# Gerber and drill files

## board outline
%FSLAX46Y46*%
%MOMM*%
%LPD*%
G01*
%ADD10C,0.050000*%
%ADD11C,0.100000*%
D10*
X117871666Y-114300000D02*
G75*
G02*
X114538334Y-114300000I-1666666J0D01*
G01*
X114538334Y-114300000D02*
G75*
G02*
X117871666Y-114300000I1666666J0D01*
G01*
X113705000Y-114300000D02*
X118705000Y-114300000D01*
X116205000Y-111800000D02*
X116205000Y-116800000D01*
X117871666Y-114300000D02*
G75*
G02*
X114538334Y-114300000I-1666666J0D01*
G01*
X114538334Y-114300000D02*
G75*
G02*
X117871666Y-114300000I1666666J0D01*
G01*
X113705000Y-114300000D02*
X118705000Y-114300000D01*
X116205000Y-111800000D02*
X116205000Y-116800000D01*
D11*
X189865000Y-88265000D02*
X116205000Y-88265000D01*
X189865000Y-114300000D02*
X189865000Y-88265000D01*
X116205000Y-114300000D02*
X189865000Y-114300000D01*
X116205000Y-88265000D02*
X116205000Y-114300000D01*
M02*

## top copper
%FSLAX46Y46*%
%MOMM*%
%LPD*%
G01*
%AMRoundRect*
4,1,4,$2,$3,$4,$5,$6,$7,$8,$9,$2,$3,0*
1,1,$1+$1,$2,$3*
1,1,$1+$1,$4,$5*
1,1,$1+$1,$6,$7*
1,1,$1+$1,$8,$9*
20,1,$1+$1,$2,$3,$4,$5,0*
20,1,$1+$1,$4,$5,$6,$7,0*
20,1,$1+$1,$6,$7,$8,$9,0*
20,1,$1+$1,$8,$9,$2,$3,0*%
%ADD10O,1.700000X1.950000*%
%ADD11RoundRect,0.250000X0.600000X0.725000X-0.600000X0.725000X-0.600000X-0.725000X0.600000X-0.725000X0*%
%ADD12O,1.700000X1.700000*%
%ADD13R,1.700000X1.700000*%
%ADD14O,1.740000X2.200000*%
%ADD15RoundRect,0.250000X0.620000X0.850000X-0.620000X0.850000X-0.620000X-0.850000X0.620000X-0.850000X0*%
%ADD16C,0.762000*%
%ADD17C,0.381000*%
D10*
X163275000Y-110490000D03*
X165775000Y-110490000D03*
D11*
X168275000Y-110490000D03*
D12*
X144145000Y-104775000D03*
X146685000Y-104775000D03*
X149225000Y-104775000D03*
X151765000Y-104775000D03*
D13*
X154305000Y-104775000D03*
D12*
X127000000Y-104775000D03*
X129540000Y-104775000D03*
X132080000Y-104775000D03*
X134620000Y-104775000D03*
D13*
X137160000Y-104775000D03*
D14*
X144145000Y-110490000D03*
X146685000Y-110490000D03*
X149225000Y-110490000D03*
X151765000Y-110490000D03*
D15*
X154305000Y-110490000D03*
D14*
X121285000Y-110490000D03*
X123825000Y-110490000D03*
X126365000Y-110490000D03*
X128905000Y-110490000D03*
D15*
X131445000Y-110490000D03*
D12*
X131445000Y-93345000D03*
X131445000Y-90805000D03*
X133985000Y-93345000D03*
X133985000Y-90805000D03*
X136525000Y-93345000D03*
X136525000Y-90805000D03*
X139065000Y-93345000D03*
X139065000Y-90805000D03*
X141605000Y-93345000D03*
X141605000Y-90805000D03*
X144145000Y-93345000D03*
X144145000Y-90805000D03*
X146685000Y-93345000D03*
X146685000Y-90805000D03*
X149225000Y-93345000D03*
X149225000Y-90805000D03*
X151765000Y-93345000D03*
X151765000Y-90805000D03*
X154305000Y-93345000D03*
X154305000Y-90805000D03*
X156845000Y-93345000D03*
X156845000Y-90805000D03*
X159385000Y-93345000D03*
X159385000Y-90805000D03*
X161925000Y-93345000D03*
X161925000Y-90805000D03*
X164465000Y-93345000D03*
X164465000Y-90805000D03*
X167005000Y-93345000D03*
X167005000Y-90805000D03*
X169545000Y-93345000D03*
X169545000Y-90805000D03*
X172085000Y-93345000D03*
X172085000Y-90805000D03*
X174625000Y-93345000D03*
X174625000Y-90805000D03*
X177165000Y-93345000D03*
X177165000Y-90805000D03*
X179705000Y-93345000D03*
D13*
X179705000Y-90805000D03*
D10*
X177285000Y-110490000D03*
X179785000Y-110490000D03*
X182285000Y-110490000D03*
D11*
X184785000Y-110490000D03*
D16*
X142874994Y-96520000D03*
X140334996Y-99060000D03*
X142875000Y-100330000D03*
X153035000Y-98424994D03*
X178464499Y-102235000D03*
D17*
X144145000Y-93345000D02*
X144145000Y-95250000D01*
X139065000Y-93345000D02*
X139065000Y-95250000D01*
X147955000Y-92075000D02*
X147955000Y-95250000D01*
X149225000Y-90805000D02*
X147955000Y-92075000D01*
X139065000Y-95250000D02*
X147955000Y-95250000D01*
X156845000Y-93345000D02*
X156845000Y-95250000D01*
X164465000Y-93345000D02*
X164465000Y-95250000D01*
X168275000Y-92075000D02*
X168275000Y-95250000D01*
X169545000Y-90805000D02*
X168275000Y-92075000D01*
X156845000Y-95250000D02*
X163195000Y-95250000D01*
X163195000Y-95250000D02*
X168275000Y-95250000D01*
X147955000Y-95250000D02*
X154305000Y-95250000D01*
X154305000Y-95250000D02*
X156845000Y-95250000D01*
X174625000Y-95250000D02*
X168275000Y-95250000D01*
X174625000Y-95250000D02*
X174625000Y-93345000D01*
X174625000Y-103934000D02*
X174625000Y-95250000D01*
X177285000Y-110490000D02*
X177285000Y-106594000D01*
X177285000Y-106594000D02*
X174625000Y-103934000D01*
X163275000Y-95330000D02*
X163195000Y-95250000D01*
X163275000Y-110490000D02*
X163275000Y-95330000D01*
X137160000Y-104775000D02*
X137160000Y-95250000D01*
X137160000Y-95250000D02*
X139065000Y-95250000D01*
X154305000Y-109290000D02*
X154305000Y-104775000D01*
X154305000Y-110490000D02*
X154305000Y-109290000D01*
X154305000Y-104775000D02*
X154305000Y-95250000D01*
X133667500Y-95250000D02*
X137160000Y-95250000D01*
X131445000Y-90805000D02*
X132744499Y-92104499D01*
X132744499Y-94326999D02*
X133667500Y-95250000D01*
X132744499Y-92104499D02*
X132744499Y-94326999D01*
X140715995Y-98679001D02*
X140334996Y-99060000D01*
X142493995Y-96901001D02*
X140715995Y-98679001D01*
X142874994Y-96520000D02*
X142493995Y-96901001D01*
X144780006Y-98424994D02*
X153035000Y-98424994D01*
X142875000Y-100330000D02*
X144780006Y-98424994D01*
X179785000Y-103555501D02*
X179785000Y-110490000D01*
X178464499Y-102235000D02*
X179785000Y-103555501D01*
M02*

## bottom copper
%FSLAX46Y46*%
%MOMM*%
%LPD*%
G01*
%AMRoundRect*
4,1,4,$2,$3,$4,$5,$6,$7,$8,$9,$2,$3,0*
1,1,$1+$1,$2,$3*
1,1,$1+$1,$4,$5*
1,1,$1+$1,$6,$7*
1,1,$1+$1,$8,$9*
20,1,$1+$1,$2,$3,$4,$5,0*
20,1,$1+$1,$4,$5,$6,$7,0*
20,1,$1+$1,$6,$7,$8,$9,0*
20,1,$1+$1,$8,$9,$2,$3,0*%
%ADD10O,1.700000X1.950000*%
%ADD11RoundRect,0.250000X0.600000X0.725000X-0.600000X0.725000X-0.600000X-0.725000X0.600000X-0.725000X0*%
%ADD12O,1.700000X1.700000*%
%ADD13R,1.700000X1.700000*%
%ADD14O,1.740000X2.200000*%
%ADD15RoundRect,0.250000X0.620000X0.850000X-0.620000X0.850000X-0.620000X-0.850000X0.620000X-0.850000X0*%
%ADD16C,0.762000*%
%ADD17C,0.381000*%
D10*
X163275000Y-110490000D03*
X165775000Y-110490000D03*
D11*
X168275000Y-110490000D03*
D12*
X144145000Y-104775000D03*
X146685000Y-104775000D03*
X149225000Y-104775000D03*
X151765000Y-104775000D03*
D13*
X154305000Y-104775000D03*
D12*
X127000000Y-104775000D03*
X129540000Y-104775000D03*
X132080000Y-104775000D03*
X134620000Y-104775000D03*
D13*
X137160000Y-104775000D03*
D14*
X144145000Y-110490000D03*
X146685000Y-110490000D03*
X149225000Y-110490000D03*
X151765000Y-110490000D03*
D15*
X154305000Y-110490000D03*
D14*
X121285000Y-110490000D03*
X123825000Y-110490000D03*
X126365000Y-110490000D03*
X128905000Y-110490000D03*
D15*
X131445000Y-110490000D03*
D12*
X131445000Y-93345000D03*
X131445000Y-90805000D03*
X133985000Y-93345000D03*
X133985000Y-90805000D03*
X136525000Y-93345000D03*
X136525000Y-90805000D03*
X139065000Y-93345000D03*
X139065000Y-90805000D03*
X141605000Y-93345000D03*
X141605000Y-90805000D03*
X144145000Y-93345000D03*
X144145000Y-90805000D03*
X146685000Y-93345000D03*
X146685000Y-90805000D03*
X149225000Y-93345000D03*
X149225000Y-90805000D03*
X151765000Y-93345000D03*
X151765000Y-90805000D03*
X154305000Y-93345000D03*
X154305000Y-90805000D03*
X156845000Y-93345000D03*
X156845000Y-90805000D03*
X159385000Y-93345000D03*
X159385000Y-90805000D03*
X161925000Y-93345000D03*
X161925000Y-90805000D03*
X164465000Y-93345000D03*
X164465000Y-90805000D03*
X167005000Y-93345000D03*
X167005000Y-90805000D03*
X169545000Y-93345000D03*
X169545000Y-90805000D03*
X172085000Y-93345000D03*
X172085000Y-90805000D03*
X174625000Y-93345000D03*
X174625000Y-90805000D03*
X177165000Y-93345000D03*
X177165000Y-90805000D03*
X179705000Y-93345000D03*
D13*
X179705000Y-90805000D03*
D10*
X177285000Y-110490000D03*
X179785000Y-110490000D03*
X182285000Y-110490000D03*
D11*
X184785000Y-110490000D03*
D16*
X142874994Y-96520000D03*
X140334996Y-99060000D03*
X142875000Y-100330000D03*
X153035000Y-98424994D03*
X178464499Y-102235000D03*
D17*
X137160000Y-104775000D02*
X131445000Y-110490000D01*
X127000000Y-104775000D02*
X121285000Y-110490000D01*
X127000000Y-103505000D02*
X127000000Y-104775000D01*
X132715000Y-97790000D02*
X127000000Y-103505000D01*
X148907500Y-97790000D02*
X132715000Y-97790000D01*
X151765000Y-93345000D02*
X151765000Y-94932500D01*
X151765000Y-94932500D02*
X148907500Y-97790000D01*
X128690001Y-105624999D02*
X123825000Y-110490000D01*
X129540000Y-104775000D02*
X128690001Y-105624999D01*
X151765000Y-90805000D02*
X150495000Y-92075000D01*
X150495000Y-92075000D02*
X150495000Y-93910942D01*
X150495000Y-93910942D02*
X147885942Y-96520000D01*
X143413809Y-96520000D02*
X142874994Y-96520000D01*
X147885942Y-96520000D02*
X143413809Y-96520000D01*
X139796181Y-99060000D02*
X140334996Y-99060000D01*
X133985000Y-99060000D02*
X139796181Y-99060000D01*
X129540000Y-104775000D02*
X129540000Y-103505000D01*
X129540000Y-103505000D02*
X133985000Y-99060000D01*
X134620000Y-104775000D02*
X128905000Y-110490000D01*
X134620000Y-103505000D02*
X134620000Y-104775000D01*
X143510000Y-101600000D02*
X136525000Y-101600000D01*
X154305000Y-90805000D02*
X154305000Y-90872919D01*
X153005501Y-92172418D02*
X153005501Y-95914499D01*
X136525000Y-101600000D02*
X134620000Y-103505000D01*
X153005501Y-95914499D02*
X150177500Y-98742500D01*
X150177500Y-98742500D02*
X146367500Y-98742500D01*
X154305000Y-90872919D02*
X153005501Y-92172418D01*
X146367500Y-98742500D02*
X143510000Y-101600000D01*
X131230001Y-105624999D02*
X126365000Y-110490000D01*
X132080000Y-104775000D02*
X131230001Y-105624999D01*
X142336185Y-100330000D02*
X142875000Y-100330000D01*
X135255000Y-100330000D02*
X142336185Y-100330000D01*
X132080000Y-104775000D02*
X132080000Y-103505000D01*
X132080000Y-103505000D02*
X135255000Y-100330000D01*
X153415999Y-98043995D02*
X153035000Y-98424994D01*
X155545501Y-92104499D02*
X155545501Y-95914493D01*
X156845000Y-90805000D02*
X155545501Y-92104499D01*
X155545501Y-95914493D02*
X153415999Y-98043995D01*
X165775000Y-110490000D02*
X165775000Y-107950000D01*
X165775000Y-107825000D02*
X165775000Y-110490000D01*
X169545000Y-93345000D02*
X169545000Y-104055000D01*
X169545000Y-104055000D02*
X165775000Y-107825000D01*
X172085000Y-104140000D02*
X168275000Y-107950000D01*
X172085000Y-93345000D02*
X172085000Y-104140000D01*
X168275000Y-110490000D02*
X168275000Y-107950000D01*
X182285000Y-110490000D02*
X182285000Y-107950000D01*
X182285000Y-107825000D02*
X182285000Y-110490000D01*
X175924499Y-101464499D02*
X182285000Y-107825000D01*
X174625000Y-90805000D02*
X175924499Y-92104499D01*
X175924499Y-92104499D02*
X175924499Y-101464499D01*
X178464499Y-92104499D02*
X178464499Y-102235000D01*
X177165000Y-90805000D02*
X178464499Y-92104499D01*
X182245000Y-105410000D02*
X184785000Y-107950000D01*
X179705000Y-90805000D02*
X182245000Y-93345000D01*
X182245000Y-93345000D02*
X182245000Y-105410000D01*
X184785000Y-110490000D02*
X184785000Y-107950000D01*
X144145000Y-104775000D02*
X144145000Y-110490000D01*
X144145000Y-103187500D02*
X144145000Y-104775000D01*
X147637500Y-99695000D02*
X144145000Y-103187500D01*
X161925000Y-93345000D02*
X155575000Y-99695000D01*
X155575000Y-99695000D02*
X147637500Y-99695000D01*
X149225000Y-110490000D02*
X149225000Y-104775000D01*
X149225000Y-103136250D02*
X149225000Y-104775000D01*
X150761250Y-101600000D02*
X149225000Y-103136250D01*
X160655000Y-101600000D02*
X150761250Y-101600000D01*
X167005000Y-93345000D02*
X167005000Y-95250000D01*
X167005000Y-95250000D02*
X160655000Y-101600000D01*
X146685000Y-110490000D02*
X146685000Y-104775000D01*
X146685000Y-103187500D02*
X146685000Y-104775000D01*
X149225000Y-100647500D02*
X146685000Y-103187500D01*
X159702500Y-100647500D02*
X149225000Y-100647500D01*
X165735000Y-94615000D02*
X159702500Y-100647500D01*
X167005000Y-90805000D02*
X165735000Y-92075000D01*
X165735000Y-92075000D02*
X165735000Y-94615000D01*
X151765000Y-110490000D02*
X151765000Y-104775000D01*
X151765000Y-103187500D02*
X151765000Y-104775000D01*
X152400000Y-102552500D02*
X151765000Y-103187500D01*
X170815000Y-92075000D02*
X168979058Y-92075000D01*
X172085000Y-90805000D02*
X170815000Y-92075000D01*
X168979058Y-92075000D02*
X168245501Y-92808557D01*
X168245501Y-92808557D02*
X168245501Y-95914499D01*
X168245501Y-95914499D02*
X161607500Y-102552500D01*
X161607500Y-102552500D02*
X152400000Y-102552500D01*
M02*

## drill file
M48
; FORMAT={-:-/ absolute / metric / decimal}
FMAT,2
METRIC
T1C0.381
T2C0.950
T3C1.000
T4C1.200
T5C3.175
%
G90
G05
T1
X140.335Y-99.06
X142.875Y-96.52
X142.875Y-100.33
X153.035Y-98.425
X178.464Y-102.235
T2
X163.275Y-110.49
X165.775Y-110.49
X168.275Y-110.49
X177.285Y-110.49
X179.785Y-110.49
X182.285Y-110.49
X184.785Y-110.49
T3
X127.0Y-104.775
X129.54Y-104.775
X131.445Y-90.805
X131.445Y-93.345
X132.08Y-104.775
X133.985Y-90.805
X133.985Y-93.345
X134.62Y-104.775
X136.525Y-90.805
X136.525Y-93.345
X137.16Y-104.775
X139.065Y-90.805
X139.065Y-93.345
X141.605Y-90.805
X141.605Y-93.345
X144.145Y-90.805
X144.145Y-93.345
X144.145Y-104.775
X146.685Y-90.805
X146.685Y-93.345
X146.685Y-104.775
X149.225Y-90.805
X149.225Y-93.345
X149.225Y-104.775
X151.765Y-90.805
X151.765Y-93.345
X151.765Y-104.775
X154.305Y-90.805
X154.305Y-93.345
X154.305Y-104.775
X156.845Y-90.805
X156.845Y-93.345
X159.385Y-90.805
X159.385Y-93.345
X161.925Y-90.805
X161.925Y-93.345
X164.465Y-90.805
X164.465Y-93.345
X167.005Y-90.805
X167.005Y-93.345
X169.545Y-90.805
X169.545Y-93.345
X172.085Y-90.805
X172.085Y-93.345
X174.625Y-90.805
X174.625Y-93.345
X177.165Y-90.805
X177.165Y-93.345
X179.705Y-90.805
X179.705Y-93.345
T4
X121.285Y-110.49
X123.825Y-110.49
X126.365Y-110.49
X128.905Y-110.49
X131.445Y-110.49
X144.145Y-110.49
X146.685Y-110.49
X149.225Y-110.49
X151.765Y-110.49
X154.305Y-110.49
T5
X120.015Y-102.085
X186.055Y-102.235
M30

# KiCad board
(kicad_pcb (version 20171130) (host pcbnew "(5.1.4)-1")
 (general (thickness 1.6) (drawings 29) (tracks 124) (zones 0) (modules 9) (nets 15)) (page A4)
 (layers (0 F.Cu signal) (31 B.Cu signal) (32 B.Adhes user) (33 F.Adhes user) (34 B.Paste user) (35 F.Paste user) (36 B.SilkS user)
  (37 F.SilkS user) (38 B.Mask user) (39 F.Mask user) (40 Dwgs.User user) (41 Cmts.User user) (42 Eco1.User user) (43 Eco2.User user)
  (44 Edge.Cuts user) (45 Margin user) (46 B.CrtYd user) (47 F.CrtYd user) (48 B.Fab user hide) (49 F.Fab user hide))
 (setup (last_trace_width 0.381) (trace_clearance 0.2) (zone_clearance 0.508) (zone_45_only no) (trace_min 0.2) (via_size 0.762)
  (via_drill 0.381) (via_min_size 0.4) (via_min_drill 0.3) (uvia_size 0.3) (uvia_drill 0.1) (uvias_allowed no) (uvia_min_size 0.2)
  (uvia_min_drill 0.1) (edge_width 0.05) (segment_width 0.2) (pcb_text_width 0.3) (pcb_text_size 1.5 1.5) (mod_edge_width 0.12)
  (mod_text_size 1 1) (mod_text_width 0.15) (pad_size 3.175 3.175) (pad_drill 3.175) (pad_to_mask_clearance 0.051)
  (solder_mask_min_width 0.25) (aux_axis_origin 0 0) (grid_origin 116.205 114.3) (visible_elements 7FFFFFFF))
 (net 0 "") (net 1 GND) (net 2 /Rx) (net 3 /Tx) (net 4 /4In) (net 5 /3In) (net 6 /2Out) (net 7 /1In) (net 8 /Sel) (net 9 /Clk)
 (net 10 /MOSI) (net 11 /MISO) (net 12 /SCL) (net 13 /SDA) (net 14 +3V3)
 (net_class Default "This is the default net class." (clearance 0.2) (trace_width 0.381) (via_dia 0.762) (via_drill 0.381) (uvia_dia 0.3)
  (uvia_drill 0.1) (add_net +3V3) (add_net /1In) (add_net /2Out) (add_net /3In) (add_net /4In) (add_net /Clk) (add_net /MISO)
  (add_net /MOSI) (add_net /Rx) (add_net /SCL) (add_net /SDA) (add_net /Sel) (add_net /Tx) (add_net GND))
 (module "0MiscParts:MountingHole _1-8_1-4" (layer F.Cu) (at 186.055 102.235 270)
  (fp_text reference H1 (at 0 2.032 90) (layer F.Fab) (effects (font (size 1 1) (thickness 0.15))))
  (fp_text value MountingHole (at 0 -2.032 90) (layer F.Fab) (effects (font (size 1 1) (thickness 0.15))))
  (pad "" np_thru_hole circle (at 0 0 270) (size 3.175 3.175) (drill 3.175) (layers *.Cu *.Mask)))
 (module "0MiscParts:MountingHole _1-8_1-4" (layer F.Cu) (at 120.015 102.085 270)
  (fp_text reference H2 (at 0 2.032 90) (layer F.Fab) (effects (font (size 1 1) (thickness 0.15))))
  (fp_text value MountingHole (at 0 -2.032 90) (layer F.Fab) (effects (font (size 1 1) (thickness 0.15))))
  (pad "" np_thru_hole circle (at 0 0 270) (size 3.175 3.175) (drill 3.175) (layers *.Cu *.Mask)))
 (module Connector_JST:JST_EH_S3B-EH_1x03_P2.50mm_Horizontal (layer F.Cu) (at 168.275 110.49 180)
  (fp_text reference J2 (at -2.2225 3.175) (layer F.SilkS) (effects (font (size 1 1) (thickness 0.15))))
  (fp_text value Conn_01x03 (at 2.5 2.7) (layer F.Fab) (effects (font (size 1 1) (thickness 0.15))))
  (pad 3 thru_hole oval (at 5 0 180) (size 1.7 1.95) (drill 0.95) (layers *.Cu *.Mask) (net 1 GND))
  (pad 2 thru_hole oval (at 2.5 0 180) (size 1.7 1.95) (drill 0.95) (layers *.Cu *.Mask) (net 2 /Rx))
  (pad 1 thru_hole roundrect (at 0 0 180) (size 1.7 1.95) (drill 0.95) (layers *.Cu *.Mask) (roundrect_rratio 0.147059) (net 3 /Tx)))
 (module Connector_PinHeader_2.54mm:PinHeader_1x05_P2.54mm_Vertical (layer F.Cu) (at 154.305 104.775 270)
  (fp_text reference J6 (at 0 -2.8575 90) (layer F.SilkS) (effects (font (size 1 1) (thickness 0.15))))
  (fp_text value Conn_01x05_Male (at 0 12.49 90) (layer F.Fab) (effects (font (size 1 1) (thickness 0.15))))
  (pad 5 thru_hole oval (at 0 10.16 270) (size 1.7 1.7) (drill 1) (layers *.Cu *.Mask) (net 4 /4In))
  (pad 4 thru_hole oval (at 0 7.62 270) (size 1.7 1.7) (drill 1) (layers *.Cu *.Mask) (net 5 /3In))
  (pad 3 thru_hole oval (at 0 5.08 270) (size 1.7 1.7) (drill 1) (layers *.Cu *.Mask) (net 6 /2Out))
  (pad 2 thru_hole oval (at 0 2.54 270) (size 1.7 1.7) (drill 1) (layers *.Cu *.Mask) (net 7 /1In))
  (pad 1 thru_hole rect (at 0 0 270) (size 1.7 1.7) (drill 1) (layers *.Cu *.Mask) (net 1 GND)))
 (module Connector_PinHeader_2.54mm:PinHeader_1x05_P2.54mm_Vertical (layer F.Cu) (at 137.16 104.775 270)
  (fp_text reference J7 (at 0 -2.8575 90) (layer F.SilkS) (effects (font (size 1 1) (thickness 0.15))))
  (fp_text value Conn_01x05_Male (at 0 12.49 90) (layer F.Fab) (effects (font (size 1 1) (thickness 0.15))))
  (pad 5 thru_hole oval (at 0 10.16 270) (size 1.7 1.7) (drill 1) (layers *.Cu *.Mask) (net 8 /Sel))
  (pad 4 thru_hole oval (at 0 7.62 270) (size 1.7 1.7) (drill 1) (layers *.Cu *.Mask) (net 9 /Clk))
  (pad 3 thru_hole oval (at 0 5.08 270) (size 1.7 1.7) (drill 1) (layers *.Cu *.Mask) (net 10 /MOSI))
  (pad 2 thru_hole oval (at 0 2.54 270) (size 1.7 1.7) (drill 1) (layers *.Cu *.Mask) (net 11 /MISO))
  (pad 1 thru_hole rect (at 0 0 270) (size 1.7 1.7) (drill 1) (layers *.Cu *.Mask) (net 1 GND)))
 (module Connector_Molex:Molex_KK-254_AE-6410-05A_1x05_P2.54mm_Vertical (layer F.Cu) (at 154.305 110.49 180)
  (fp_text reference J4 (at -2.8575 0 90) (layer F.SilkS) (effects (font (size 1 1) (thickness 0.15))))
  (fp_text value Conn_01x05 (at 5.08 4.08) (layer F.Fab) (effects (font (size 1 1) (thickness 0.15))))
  (pad 5 thru_hole oval (at 10.16 0 180) (size 1.74 2.2) (drill 1.2) (layers *.Cu *.Mask) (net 4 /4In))
  (pad 4 thru_hole oval (at 7.62 0 180) (size 1.74 2.2) (drill 1.2) (layers *.Cu *.Mask) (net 5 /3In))
  (pad 3 thru_hole oval (at 5.08 0 180) (size 1.74 2.2) (drill 1.2) (layers *.Cu *.Mask) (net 6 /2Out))
  (pad 2 thru_hole oval (at 2.54 0 180) (size 1.74 2.2) (drill 1.2) (layers *.Cu *.Mask) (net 7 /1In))
  (pad 1 thru_hole roundrect (at 0 0 180) (size 1.74 2.2) (drill 1.2) (layers *.Cu *.Mask) (roundrect_rratio 0.143678) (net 1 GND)))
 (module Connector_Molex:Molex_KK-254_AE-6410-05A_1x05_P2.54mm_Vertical (layer F.Cu) (at 131.445 110.49 180)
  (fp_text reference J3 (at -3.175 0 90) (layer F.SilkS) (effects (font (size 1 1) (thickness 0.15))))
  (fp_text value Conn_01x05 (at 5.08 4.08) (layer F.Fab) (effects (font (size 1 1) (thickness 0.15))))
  (pad 5 thru_hole oval (at 10.16 0 180) (size 1.74 2.2) (drill 1.2) (layers *.Cu *.Mask) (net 8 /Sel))
  (pad 4 thru_hole oval (at 7.62 0 180) (size 1.74 2.2) (drill 1.2) (layers *.Cu *.Mask) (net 9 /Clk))
  (pad 3 thru_hole oval (at 5.08 0 180) (size 1.74 2.2) (drill 1.2) (layers *.Cu *.Mask) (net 10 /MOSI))
  (pad 2 thru_hole oval (at 2.54 0 180) (size 1.74 2.2) (drill 1.2) (layers *.Cu *.Mask) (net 11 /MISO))
  (pad 1 thru_hole roundrect (at 0 0 180) (size 1.74 2.2) (drill 1.2) (layers *.Cu *.Mask) (roundrect_rratio 0.143678) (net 1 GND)))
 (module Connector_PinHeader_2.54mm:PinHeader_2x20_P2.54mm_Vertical (layer F.Cu) (at 179.705 90.805 270)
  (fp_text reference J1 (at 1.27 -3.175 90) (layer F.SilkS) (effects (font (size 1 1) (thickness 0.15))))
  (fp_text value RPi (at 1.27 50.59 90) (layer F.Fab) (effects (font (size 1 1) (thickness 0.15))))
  (pad 40 thru_hole oval (at 2.54 48.26 270) (size 1.7 1.7) (drill 1) (layers *.Cu *.Mask))
  (pad 39 thru_hole oval (at 0 48.26 270) (size 1.7 1.7) (drill 1) (layers *.Cu *.Mask) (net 1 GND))
  (pad 38 thru_hole oval (at 2.54 45.72 270) (size 1.7 1.7) (drill 1) (layers *.Cu *.Mask))
  (pad 37 thru_hole oval (at 0 45.72 270) (size 1.7 1.7) (drill 1) (layers *.Cu *.Mask))
  (pad 36 thru_hole oval (at 2.54 43.18 270) (size 1.7 1.7) (drill 1) (layers *.Cu *.Mask))
  (pad 35 thru_hole oval (at 0 43.18 270) (size 1.7 1.7) (drill 1) (layers *.Cu *.Mask))
  (pad 34 thru_hole oval (at 2.54 40.64 270) (size 1.7 1.7) (drill 1) (layers *.Cu *.Mask) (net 1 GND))
  (pad 33 thru_hole oval (at 0 40.64 270) (size 1.7 1.7) (drill 1) (layers *.Cu *.Mask))
  (pad 32 thru_hole oval (at 2.54 38.1 270) (size 1.7 1.7) (drill 1) (layers *.Cu *.Mask))
  (pad 31 thru_hole oval (at 0 38.1 270) (size 1.7 1.7) (drill 1) (layers *.Cu *.Mask))
  (pad 30 thru_hole oval (at 2.54 35.56 270) (size 1.7 1.7) (drill 1) (layers *.Cu *.Mask) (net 1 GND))
  (pad 29 thru_hole oval (at 0 35.56 270) (size 1.7 1.7) (drill 1) (layers *.Cu *.Mask))
  (pad 28 thru_hole oval (at 2.54 33.02 270) (size 1.7 1.7) (drill 1) (layers *.Cu *.Mask))
  (pad 27 thru_hole oval (at 0 33.02 270) (size 1.7 1.7) (drill 1) (layers *.Cu *.Mask))
  (pad 26 thru_hole oval (at 2.54 30.48 270) (size 1.7 1.7) (drill 1) (layers *.Cu *.Mask))
  (pad 25 thru_hole oval (at 0 30.48 270) (size 1.7 1.7) (drill 1) (layers *.Cu *.Mask) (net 1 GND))
  (pad 24 thru_hole oval (at 2.54 27.94 270) (size 1.7 1.7) (drill 1) (layers *.Cu *.Mask) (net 8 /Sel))
  (pad 23 thru_hole oval (at 0 27.94 270) (size 1.7 1.7) (drill 1) (layers *.Cu *.Mask) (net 9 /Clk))
  (pad 22 thru_hole oval (at 2.54 25.4 270) (size 1.7 1.7) (drill 1) (layers *.Cu *.Mask))
  (pad 21 thru_hole oval (at 0 25.4 270) (size 1.7 1.7) (drill 1) (layers *.Cu *.Mask) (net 11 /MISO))
  (pad 20 thru_hole oval (at 2.54 22.86 270) (size 1.7 1.7) (drill 1) (layers *.Cu *.Mask) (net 1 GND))
  (pad 19 thru_hole oval (at 0 22.86 270) (size 1.7 1.7) (drill 1) (layers *.Cu *.Mask) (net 10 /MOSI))
  (pad 18 thru_hole oval (at 2.54 20.32 270) (size 1.7 1.7) (drill 1) (layers *.Cu *.Mask))
  (pad 17 thru_hole oval (at 0 20.32 270) (size 1.7 1.7) (drill 1) (layers *.Cu *.Mask))
  (pad 16 thru_hole oval (at 2.54 17.78 270) (size 1.7 1.7) (drill 1) (layers *.Cu *.Mask) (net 4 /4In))
  (pad 15 thru_hole oval (at 0 17.78 270) (size 1.7 1.7) (drill 1) (layers *.Cu *.Mask))
  (pad 14 thru_hole oval (at 2.54 15.24 270) (size 1.7 1.7) (drill 1) (layers *.Cu *.Mask) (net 1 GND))
  (pad 13 thru_hole oval (at 0 15.24 270) (size 1.7 1.7) (drill 1) (layers *.Cu *.Mask))
  (pad 12 thru_hole oval (at 2.54 12.7 270) (size 1.7 1.7) (drill 1) (layers *.Cu *.Mask) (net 6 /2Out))
  (pad 11 thru_hole oval (at 0 12.7 270) (size 1.7 1.7) (drill 1) (layers *.Cu *.Mask) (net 5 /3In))
  (pad 10 thru_hole oval (at 2.54 10.16 270) (size 1.7 1.7) (drill 1) (layers *.Cu *.Mask) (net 2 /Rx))
  (pad 9 thru_hole oval (at 0 10.16 270) (size 1.7 1.7) (drill 1) (layers *.Cu *.Mask) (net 1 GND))
  (pad 8 thru_hole oval (at 2.54 7.62 270) (size 1.7 1.7) (drill 1) (layers *.Cu *.Mask) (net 3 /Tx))
  (pad 7 thru_hole oval (at 0 7.62 270) (size 1.7 1.7) (drill 1) (layers *.Cu *.Mask) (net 7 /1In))
  (pad 6 thru_hole oval (at 2.54 5.08 270) (size 1.7 1.7) (drill 1) (layers *.Cu *.Mask) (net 1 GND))
  (pad 5 thru_hole oval (at 0 5.08 270) (size 1.7 1.7) (drill 1) (layers *.Cu *.Mask) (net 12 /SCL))
  (pad 4 thru_hole oval (at 2.54 2.54 270) (size 1.7 1.7) (drill 1) (layers *.Cu *.Mask))
  (pad 3 thru_hole oval (at 0 2.54 270) (size 1.7 1.7) (drill 1) (layers *.Cu *.Mask) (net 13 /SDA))
  (pad 2 thru_hole oval (at 2.54 0 270) (size 1.7 1.7) (drill 1) (layers *.Cu *.Mask))
  (pad 1 thru_hole rect (at 0 0 270) (size 1.7 1.7) (drill 1) (layers *.Cu *.Mask) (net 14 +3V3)))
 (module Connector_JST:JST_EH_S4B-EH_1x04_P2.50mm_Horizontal (layer F.Cu) (at 184.785 110.49 180)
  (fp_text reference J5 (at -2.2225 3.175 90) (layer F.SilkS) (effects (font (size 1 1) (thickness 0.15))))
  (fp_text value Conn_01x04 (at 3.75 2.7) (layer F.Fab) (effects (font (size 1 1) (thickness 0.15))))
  (pad 4 thru_hole oval (at 7.5 0 180) (size 1.7 1.95) (drill 0.95) (layers *.Cu *.Mask) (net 1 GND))
  (pad 3 thru_hole oval (at 5 0 180) (size 1.7 1.95) (drill 0.95) (layers *.Cu *.Mask) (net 13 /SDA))
  (pad 2 thru_hole oval (at 2.5 0 180) (size 1.7 1.95) (drill 0.95) (layers *.Cu *.Mask) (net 12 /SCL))
  (pad 1 thru_hole roundrect (at 0 0 180) (size 1.7 1.95) (drill 0.95) (layers *.Cu *.Mask) (roundrect_rratio 0.147059) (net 14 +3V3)))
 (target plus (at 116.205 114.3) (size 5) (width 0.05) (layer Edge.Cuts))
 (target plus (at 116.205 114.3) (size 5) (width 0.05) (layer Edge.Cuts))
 (gr_line (start 189.865 88.265) (end 116.205 88.265) (layer Edge.Cuts) (width 0.1))
 (gr_line (start 189.865 114.3) (end 189.865 88.265) (layer Edge.Cuts) (width 0.1))
 (gr_line (start 116.205 114.3) (end 189.865 114.3) (layer Edge.Cuts) (width 0.1))
 (gr_line (start 116.205 88.265) (end 116.205 114.3) (layer Edge.Cuts) (width 0.1))
 (segment (start 144.145 93.345) (end 144.145 95.25) (width 0.381) (layer F.Cu) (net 1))
 (segment (start 139.065 93.345) (end 139.065 95.25) (width 0.381) (layer F.Cu) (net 1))
 (segment (start 147.955 92.075) (end 147.955 95.25) (width 0.381) (layer F.Cu) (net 1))
 (segment (start 149.225 90.805) (end 147.955 92.075) (width 0.381) (layer F.Cu) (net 1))
 (segment (start 139.065 95.25) (end 147.955 95.25) (width 0.381) (layer F.Cu) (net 1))
 (segment (start 156.845 93.345) (end 156.845 95.25) (width 0.381) (layer F.Cu) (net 1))
 (segment (start 164.465 93.345) (end 164.465 95.25) (width 0.381) (layer F.Cu) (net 1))
 (segment (start 168.275 92.075) (end 168.275 95.25) (width 0.381) (layer F.Cu) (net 1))
 (segment (start 169.545 90.805) (end 168.275 92.075) (width 0.381) (layer F.Cu) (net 1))
 (segment (start 156.845 95.25) (end 163.195 95.25) (width 0.381) (layer F.Cu) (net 1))
 (segment (start 163.195 95.25) (end 168.275 95.25) (width 0.381) (layer F.Cu) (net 1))
 (segment (start 147.955 95.25) (end 154.305 95.25) (width 0.381) (layer F.Cu) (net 1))
 (segment (start 154.305 95.25) (end 156.845 95.25) (width 0.381) (layer F.Cu) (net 1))
 (segment (start 174.625 95.25) (end 168.275 95.25) (width 0.381) (layer F.Cu) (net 1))
 (segment (start 174.625 95.25) (end 174.625 93.345) (width 0.381) (layer F.Cu) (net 1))
 (segment (start 174.625 103.934) (end 174.625 95.25) (width 0.381) (layer F.Cu) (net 1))
 (segment (start 177.285 110.49) (end 177.285 106.594) (width 0.381) (layer F.Cu) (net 1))
 (segment (start 177.285 106.594) (end 174.625 103.934) (width 0.381) (layer F.Cu) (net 1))
 (segment (start 163.275 95.33) (end 163.195 95.25) (width 0.381) (layer F.Cu) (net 1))
 (segment (start 163.275 110.49) (end 163.275 95.33) (width 0.381) (layer F.Cu) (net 1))
 (segment (start 137.16 104.775) (end 131.445 110.49) (width 0.381) (layer B.Cu) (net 1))
 (segment (start 137.16 104.775) (end 137.16 95.25) (width 0.381) (layer F.Cu) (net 1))
 (segment (start 137.16 95.25) (end 139.065 95.25) (width 0.381) (layer F.Cu) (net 1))
 (segment (start 154.305 109.29) (end 154.305 104.775) (width 0.381) (layer F.Cu) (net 1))
 (segment (start 154.305 110.49) (end 154.305 109.29) (width 0.381) (layer F.Cu) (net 1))
 (segment (start 154.305 104.775) (end 154.305 95.25) (width 0.381) (layer F.Cu) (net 1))
 (segment (start 133.6675 95.25) (end 137.16 95.25) (width 0.381) (layer F.Cu) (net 1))
 (segment (start 131.445 90.805) (end 132.744499 92.104499) (width 0.381) (layer F.Cu) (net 1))
 (segment (start 132.744499 94.326999) (end 133.6675 95.25) (width 0.381) (layer F.Cu) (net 1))
 (segment (start 132.744499 92.104499) (end 132.744499 94.326999) (width 0.381) (layer F.Cu) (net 1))
 (segment (start 127 104.775) (end 121.285 110.49) (width 0.381) (layer B.Cu) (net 8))
 (segment (start 127 103.505) (end 127 104.775) (width 0.381) (layer B.Cu) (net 8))
 (segment (start 132.715 97.79) (end 127 103.505) (width 0.381) (layer B.Cu) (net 8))
 (segment (start 148.9075 97.79) (end 132.715 97.79) (width 0.381) (layer B.Cu) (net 8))
 (segment (start 151.765 93.345) (end 151.765 94.9325) (width 0.381) (layer B.Cu) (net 8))
 (segment (start 151.765 94.9325) (end 148.9075 97.79) (width 0.381) (layer B.Cu) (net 8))
 (segment (start 128.690001 105.624999) (end 123.825 110.49) (width 0.381) (layer B.Cu) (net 9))
 (segment (start 129.54 104.775) (end 128.690001 105.624999) (width 0.381) (layer B.Cu) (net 9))
 (via (at 142.874994 96.52) (size 0.762) (drill 0.381) (layers F.Cu B.Cu) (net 9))
 (segment (start 151.765 90.805) (end 150.495 92.075) (width 0.381) (layer B.Cu) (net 9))
 (segment (start 150.495 92.075) (end 150.495 93.910942) (width 0.381) (layer B.Cu) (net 9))
 (segment (start 150.495 93.910942) (end 147.885942 96.52) (width 0.381) (layer B.Cu) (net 9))
 (segment (start 143.413809 96.52) (end 142.874994 96.52) (width 0.381) (layer B.Cu) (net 9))
 (segment (start 147.885942 96.52) (end 143.413809 96.52) (width 0.381) (layer B.Cu) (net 9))
 (segment (start 140.715995 98.679001) (end 140.334996 99.06) (width 0.381) (layer F.Cu) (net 9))
 (segment (start 142.493995 96.901001) (end 140.715995 98.679001) (width 0.381) (layer F.Cu) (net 9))
 (via (at 140.334996 99.06) (size 0.762) (drill 0.381) (layers F.Cu B.Cu) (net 9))
 (segment (start 142.874994 96.52) (end 142.493995 96.901001) (width 0.381) (layer F.Cu) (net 9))
 (segment (start 139.796181 99.06) (end 140.334996 99.06) (width 0.381) (layer B.Cu) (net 9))
 (segment (start 133.985 99.06) (end 139.796181 99.06) (width 0.381) (layer B.Cu) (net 9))
 (segment (start 129.54 104.775) (end 129.54 103.505) (width 0.381) (layer B.Cu) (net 9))
 (segment (start 129.54 103.505) (end 133.985 99.06) (width 0.381) (layer B.Cu) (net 9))
 (segment (start 134.62 104.775) (end 128.905 110.49) (width 0.381) (layer B.Cu) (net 11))
 (segment (start 134.62 103.505) (end 134.62 104.775) (width 0.381) (layer B.Cu) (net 11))
 (segment (start 143.51 101.6) (end 136.525 101.6) (width 0.381) (layer B.Cu) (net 11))
 (segment (start 154.305 90.805) (end 154.305 90.872919) (width 0.381) (layer B.Cu) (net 11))
 (segment (start 153.005501 92.172418) (end 153.005501 95.914499) (width 0.381) (layer B.Cu) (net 11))
 (segment (start 136.525 101.6) (end 134.62 103.505) (width 0.381) (layer B.Cu) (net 11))
 (segment (start 153.005501 95.914499) (end 150.1775 98.7425) (width 0.381) (layer B.Cu) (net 11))
 (segment (start 150.1775 98.7425) (end 146.3675 98.7425) (width 0.381) (layer B.Cu) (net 11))
 (segment (start 154.305 90.872919) (end 153.005501 92.172418) (width 0.381) (layer B.Cu) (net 11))
 (segment (start 146.3675 98.7425) (end 143.51 101.6) (width 0.381) (layer B.Cu) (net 11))
 (segment (start 131.230001 105.624999) (end 126.365 110.49) (width 0.381) (layer B.Cu) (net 10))
 (segment (start 132.08 104.775) (end 131.230001 105.624999) (width 0.381) (layer B.Cu) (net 10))
 (via (at 142.875 100.33) (size 0.762) (drill 0.381) (layers F.Cu B.Cu) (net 10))
 (segment (start 142.336185 100.33) (end 142.875 100.33) (width 0.381) (layer B.Cu) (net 10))
 (segment (start 135.255 100.33) (end 142.336185 100.33) (width 0.381) (layer B.Cu) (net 10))
 (segment (start 132.08 104.775) (end 132.08 103.505) (width 0.381) (layer B.Cu) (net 10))
 (segment (start 132.08 103.505) (end 135.255 100.33) (width 0.381) (layer B.Cu) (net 10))
 (segment (start 153.415999 98.043995) (end 153.035 98.424994) (width 0.381) (layer B.Cu) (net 10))
 (segment (start 155.545501 92.104499) (end 155.545501 95.914493) (width 0.381) (layer B.Cu) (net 10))
 (segment (start 156.845 90.805) (end 155.545501 92.104499) (width 0.381) (layer B.Cu) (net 10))
 (segment (start 155.545501 95.914493) (end 153.415999 98.043995) (width 0.381) (layer B.Cu) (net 10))
 (via (at 153.035 98.424994) (size 0.762) (drill 0.381) (layers F.Cu B.Cu) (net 10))
 (segment (start 144.780006 98.424994) (end 153.035 98.424994) (width 0.381) (layer F.Cu) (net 10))
 (segment (start 142.875 100.33) (end 144.780006 98.424994) (width 0.381) (layer F.Cu) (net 10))
 (segment (start 165.775 110.49) (end 165.775 107.95) (width 0.381) (layer B.Cu) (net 2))
 (segment (start 165.775 107.825) (end 165.775 110.49) (width 0.381) (layer B.Cu) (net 2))
 (segment (start 169.545 93.345) (end 169.545 104.055) (width 0.381) (layer B.Cu) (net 2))
 (segment (start 169.545 104.055) (end 165.775 107.825) (width 0.381) (layer B.Cu) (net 2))
 (segment (start 172.085 104.14) (end 168.275 107.95) (width 0.381) (layer B.Cu) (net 3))
 (segment (start 172.085 93.345) (end 172.085 104.14) (width 0.381) (layer B.Cu) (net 3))
 (segment (start 168.275 110.49) (end 168.275 107.95) (width 0.381) (layer B.Cu) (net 3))
 (segment (start 182.285 110.49) (end 182.285 107.95) (width 0.381) (layer B.Cu) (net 12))
 (segment (start 182.285 107.825) (end 182.285 110.49) (width 0.381) (layer B.Cu) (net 12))
 (segment (start 175.924499 101.464499) (end 182.285 107.825) (width 0.381) (layer B.Cu) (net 12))
 (segment (start 174.625 90.805) (end 175.924499 92.104499) (width 0.381) (layer B.Cu) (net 12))
 (segment (start 175.924499 92.104499) (end 175.924499 101.464499) (width 0.381) (layer B.Cu) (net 12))
 (via (at 178.464499 102.235) (size 0.762) (drill 0.381) (layers F.Cu B.Cu) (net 13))
 (segment (start 178.464499 92.104499) (end 178.464499 102.235) (width 0.381) (layer B.Cu) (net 13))
 (segment (start 177.165 90.805) (end 178.464499 92.104499) (width 0.381) (layer B.Cu) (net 13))
 (segment (start 179.785 103.555501) (end 179.785 110.49) (width 0.381) (layer F.Cu) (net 13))
 (segment (start 178.464499 102.235) (end 179.785 103.555501) (width 0.381) (layer F.Cu) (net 13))
 (segment (start 182.245 105.41) (end 184.785 107.95) (width 0.381) (layer B.Cu) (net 14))
 (segment (start 179.705 90.805) (end 182.245 93.345) (width 0.381) (layer B.Cu) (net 14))
 (segment (start 182.245 93.345) (end 182.245 105.41) (width 0.381) (layer B.Cu) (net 14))
 (segment (start 184.785 110.49) (end 184.785 107.95) (width 0.381) (layer B.Cu) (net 14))
 (segment (start 144.145 104.775) (end 144.145 110.49) (width 0.381) (layer B.Cu) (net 4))
 (segment (start 144.145 103.1875) (end 144.145 104.775) (width 0.381) (layer B.Cu) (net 4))
 (segment (start 147.6375 99.695) (end 144.145 103.1875) (width 0.381) (layer B.Cu) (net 4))
 (segment (start 161.925 93.345) (end 155.575 99.695) (width 0.381) (layer B.Cu) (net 4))
 (segment (start 155.575 99.695) (end 147.6375 99.695) (width 0.381) (layer B.Cu) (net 4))
 (segment (start 149.225 110.49) (end 149.225 104.775) (width 0.381) (layer B.Cu) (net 6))
 (segment (start 149.225 103.13625) (end 149.225 104.775) (width 0.381) (layer B.Cu) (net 6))
 (segment (start 150.76125 101.6) (end 149.225 103.13625) (width 0.381) (layer B.Cu) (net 6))
 (segment (start 160.655 101.6) (end 150.76125 101.6) (width 0.381) (layer B.Cu) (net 6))
 (segment (start 167.005 93.345) (end 167.005 95.25) (width 0.381) (layer B.Cu) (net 6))
 (segment (start 167.005 95.25) (end 160.655 101.6) (width 0.381) (layer B.Cu) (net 6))
 (segment (start 146.685 110.49) (end 146.685 104.775) (width 0.381) (layer B.Cu) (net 5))
 (segment (start 146.685 103.1875) (end 146.685 104.775) (width 0.381) (layer B.Cu) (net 5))
 (segment (start 149.225 100.6475) (end 146.685 103.1875) (width 0.381) (layer B.Cu) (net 5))
 (segment (start 159.7025 100.6475) (end 149.225 100.6475) (width 0.381) (layer B.Cu) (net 5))
 (segment (start 165.735 94.615) (end 159.7025 100.6475) (width 0.381) (layer B.Cu) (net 5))
 (segment (start 167.005 90.805) (end 165.735 92.075) (width 0.381) (layer B.Cu) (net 5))
 (segment (start 165.735 92.075) (end 165.735 94.615) (width 0.381) (layer B.Cu) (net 5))
 (segment (start 151.765 110.49) (end 151.765 104.775) (width 0.381) (layer B.Cu) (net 7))
 (segment (start 151.765 103.1875) (end 151.765 104.775) (width 0.381) (layer B.Cu) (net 7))
 (segment (start 152.4 102.5525) (end 151.765 103.1875) (width 0.381) (layer B.Cu) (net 7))
 (segment (start 170.815 92.075) (end 168.979058 92.075) (width 0.381) (layer B.Cu) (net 7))
 (segment (start 172.085 90.805) (end 170.815 92.075) (width 0.381) (layer B.Cu) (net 7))
 (segment (start 168.979058 92.075) (end 168.245501 92.808557) (width 0.381) (layer B.Cu) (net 7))
 (segment (start 168.245501 92.808557) (end 168.245501 95.914499) (width 0.381) (layer B.Cu) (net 7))
 (segment (start 168.245501 95.914499) (end 161.6075 102.5525) (width 0.381) (layer B.Cu) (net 7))
 (segment (start 161.6075 102.5525) (end 152.4 102.5525) (width 0.381) (layer B.Cu) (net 7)))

